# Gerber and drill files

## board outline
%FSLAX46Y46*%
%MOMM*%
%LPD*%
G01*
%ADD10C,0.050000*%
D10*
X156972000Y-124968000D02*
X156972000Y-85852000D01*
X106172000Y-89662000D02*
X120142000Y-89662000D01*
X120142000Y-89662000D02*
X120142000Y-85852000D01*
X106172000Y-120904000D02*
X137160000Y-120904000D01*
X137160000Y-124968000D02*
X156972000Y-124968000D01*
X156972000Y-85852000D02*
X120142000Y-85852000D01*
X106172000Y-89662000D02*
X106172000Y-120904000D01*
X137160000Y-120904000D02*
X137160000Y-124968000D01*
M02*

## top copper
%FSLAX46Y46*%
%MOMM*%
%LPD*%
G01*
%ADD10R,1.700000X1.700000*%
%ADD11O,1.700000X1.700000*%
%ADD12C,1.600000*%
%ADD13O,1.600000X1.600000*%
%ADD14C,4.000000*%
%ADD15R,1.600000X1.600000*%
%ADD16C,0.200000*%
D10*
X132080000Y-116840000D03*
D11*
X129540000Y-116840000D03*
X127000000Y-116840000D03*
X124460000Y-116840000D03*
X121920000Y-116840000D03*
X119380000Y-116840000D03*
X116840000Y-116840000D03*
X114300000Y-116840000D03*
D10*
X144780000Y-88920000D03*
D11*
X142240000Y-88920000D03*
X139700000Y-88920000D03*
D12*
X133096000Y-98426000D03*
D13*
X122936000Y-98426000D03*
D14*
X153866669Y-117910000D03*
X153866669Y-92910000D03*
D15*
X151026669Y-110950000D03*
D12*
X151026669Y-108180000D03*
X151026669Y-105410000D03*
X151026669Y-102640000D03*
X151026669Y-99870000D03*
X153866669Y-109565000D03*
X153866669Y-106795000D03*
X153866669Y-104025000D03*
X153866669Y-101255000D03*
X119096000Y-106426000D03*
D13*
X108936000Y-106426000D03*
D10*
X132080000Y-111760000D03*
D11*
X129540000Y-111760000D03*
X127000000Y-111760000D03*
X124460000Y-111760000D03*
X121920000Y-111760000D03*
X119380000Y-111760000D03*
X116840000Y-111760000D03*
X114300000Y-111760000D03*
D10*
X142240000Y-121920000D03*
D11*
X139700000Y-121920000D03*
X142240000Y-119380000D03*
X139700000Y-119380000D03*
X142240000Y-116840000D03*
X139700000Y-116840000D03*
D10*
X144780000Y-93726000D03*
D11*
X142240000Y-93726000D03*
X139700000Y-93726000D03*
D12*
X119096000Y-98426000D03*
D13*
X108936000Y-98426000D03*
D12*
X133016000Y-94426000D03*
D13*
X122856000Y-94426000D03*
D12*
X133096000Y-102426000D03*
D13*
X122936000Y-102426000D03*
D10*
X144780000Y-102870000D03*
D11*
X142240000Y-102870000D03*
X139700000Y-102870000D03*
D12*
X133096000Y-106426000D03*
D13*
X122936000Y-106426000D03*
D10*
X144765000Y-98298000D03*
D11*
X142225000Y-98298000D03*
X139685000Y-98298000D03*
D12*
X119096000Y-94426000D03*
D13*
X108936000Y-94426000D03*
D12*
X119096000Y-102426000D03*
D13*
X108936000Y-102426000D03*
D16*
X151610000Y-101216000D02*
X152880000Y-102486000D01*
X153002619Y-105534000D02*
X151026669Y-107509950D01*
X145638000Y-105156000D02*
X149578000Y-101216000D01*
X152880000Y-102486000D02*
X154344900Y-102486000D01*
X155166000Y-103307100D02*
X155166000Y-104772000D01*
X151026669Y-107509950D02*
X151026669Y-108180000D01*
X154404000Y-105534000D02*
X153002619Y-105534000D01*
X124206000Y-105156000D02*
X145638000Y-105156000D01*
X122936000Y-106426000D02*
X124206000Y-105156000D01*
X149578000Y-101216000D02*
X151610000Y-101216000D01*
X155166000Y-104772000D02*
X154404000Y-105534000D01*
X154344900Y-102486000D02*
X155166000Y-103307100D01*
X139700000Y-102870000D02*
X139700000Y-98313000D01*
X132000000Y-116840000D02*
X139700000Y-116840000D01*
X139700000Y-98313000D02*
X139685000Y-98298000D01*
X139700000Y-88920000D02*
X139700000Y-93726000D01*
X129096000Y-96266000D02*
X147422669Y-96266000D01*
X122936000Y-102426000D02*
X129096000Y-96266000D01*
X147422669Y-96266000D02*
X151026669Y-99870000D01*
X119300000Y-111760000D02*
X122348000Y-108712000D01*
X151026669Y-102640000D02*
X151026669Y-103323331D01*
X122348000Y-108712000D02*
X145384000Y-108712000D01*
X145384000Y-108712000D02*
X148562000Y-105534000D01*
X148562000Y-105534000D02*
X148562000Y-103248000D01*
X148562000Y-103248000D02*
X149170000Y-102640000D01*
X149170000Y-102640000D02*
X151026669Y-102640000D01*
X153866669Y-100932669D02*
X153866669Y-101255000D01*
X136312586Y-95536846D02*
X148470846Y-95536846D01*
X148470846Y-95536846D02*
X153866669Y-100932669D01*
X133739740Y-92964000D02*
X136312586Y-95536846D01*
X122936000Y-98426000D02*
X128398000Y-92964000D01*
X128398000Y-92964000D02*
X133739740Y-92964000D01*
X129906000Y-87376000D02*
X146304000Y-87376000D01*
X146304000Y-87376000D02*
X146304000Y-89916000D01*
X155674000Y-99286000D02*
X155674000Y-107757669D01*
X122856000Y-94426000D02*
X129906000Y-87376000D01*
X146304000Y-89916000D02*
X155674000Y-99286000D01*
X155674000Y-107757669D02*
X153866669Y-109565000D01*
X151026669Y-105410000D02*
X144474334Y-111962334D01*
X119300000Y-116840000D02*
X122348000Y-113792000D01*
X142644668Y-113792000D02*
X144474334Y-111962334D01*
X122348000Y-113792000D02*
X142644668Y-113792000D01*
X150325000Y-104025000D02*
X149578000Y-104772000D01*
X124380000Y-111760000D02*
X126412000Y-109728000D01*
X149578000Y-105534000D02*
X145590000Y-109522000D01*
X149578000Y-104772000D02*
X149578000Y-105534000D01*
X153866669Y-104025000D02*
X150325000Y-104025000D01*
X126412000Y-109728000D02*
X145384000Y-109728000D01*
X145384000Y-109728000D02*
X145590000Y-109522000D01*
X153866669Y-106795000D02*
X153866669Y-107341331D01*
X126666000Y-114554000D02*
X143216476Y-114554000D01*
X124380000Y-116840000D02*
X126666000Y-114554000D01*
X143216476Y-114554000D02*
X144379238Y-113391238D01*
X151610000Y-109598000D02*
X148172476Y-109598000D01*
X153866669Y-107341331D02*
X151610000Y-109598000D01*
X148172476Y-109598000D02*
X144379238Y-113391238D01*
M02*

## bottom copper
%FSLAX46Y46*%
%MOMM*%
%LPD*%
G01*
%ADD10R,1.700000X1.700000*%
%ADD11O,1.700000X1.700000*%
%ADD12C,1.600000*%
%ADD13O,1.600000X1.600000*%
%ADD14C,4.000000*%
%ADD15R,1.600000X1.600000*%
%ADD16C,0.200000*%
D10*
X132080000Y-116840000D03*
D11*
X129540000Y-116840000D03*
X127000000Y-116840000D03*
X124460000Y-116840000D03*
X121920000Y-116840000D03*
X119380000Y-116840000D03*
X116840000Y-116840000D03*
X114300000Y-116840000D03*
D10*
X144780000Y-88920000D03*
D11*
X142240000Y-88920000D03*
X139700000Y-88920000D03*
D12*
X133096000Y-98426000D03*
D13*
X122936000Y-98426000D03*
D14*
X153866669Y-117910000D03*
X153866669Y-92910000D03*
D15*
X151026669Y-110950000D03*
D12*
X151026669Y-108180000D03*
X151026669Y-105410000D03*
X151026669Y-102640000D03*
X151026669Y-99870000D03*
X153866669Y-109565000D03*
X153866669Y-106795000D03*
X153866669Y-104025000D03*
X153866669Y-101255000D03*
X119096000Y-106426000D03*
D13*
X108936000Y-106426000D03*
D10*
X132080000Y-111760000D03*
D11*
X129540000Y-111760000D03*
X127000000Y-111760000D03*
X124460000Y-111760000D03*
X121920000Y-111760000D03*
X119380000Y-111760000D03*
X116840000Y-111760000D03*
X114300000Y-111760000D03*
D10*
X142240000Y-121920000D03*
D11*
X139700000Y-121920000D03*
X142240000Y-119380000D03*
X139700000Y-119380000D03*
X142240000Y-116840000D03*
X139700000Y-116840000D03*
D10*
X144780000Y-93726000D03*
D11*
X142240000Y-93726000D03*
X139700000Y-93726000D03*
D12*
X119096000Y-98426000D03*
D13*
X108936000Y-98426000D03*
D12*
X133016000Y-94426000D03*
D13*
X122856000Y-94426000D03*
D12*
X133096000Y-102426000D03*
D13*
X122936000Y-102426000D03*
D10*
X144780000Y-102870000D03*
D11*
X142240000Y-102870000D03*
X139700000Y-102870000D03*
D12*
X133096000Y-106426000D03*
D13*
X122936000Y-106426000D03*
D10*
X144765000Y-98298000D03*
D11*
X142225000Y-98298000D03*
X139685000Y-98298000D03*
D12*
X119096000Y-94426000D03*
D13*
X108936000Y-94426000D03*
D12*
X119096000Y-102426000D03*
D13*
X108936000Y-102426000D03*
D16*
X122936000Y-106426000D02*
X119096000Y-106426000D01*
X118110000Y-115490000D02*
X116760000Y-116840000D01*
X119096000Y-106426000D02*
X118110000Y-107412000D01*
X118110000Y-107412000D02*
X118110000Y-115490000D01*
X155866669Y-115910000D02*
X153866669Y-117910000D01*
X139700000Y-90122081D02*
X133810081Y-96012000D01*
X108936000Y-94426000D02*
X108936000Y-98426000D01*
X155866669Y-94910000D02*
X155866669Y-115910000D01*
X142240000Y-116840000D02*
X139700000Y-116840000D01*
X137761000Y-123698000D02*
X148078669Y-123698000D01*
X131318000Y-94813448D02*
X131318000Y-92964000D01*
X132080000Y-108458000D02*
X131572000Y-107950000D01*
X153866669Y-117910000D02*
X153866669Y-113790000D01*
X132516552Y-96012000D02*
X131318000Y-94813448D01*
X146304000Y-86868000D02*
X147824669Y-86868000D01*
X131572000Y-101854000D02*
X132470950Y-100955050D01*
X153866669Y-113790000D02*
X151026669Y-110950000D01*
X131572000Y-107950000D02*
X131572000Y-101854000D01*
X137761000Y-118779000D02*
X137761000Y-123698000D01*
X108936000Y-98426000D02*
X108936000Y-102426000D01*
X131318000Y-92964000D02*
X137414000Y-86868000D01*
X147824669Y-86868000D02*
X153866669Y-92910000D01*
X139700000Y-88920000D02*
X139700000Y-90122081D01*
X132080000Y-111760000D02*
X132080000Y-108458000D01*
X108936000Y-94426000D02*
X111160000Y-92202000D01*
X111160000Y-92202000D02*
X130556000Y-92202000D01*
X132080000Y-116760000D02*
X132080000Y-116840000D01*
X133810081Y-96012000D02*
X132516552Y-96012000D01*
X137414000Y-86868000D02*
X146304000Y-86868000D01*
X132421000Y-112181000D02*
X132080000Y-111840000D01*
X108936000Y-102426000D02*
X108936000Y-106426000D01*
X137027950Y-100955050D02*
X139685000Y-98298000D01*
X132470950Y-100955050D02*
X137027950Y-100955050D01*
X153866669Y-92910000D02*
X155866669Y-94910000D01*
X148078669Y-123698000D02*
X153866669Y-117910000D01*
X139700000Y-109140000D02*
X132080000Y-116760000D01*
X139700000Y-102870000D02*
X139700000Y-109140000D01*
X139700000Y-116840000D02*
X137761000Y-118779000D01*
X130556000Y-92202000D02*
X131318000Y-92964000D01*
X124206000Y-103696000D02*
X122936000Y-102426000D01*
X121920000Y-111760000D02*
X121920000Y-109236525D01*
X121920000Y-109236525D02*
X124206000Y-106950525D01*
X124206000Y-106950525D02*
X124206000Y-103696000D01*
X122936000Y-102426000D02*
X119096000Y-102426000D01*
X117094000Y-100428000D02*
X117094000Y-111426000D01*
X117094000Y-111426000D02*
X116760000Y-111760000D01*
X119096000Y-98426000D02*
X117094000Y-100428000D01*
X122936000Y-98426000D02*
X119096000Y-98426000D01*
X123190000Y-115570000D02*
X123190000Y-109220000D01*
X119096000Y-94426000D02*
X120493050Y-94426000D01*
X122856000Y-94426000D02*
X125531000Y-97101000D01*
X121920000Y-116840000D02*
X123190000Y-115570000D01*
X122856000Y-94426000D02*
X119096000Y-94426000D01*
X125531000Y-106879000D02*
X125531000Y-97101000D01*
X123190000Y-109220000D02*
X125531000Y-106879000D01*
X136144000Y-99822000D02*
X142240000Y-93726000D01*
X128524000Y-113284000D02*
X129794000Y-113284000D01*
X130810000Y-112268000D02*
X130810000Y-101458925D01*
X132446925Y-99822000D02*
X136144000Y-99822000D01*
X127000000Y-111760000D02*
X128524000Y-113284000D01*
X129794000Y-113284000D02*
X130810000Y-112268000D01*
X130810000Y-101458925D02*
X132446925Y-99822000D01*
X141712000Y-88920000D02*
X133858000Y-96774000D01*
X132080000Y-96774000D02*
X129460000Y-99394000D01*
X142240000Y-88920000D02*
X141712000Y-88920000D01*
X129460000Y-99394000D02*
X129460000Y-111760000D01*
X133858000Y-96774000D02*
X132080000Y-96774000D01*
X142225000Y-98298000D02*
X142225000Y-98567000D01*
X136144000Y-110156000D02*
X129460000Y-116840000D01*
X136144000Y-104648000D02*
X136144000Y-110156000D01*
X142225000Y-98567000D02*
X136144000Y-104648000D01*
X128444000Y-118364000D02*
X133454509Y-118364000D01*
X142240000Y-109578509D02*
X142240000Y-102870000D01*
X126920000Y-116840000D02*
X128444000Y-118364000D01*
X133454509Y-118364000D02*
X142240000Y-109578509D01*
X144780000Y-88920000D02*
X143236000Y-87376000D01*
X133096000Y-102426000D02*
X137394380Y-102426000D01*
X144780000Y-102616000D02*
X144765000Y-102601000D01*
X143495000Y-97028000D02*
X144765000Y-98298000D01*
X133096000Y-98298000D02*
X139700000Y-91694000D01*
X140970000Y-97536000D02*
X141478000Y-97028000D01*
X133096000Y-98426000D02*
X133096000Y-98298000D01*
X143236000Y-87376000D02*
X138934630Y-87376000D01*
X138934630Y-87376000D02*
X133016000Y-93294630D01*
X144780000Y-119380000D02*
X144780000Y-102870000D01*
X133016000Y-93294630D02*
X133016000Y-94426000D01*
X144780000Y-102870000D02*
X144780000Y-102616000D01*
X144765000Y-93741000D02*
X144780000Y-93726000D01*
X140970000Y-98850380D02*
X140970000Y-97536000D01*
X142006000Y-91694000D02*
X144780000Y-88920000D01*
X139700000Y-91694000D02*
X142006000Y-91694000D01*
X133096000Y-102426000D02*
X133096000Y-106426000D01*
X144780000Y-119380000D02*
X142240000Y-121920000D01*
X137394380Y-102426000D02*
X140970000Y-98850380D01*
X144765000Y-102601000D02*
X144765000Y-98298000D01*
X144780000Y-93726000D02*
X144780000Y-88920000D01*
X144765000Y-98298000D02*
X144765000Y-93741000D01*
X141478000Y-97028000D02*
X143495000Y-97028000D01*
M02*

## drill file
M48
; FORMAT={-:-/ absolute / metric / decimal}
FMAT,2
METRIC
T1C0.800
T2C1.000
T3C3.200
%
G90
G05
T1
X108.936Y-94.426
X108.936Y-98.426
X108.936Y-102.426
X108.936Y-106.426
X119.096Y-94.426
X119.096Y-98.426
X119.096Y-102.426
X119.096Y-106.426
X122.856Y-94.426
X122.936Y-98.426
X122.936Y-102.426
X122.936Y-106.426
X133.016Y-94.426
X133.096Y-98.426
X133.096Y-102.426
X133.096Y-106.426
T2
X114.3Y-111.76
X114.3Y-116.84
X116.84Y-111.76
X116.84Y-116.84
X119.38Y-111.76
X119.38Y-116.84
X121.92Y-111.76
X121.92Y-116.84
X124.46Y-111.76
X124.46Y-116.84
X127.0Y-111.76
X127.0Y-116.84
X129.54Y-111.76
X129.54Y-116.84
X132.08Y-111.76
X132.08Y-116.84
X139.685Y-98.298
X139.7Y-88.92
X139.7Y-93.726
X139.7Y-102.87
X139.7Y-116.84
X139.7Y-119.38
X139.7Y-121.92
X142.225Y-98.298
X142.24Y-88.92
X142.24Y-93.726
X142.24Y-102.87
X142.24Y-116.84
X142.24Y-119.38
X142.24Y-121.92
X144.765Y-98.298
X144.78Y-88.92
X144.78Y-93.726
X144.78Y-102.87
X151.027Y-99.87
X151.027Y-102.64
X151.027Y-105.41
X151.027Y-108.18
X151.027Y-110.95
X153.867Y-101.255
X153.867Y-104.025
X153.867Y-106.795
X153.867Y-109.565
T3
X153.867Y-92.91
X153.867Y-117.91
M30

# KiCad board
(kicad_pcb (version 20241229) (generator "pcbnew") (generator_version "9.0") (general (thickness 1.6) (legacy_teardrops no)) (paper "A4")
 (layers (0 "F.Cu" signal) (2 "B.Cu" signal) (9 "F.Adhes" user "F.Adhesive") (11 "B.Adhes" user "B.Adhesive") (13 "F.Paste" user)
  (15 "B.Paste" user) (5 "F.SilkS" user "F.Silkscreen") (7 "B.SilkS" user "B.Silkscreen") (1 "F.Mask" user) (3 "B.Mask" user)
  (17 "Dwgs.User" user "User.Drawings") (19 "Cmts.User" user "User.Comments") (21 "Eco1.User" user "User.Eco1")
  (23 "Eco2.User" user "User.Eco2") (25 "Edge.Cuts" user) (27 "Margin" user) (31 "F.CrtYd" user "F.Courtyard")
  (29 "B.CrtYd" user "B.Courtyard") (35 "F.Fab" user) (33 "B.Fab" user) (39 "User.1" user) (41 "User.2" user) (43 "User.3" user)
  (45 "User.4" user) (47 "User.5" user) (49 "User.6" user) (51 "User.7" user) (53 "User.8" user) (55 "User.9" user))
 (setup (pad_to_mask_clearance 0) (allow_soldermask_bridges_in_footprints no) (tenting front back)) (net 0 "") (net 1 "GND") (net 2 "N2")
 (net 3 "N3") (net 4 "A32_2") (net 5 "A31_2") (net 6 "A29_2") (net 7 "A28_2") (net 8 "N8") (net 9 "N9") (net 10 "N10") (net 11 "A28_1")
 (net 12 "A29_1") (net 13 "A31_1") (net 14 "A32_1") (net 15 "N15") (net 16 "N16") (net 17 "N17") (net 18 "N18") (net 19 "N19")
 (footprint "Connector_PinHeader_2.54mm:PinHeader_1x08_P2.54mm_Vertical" (layer "F.Cu") (at 132.08 116.84 -90)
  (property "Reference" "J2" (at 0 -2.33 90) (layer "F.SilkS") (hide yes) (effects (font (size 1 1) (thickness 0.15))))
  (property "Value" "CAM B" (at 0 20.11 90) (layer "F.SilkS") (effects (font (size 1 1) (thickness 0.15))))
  (pad "1" thru_hole rect (at 0 0 270) (size 1.7 1.7) (drill 1) (layers "*.Cu" "*.Mask") (remove_unused_layers no) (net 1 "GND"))
  (pad "2" thru_hole oval (at 0 2.54 270) (size 1.7 1.7) (drill 1) (layers "*.Cu" "*.Mask") (remove_unused_layers no) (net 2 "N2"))
  (pad "3" thru_hole oval (at 0 5.08 270) (size 1.7 1.7) (drill 1) (layers "*.Cu" "*.Mask") (remove_unused_layers no) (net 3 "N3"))
  (pad "4" thru_hole oval (at 0 7.62 270) (size 1.7 1.7) (drill 1) (layers "*.Cu" "*.Mask") (remove_unused_layers no) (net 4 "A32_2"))
  (pad "5" thru_hole oval (at 0 10.16 270) (size 1.7 1.7) (drill 1) (layers "*.Cu" "*.Mask") (remove_unused_layers no) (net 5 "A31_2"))
  (pad "6" thru_hole oval (at 0 12.7 270) (size 1.7 1.7) (drill 1) (layers "*.Cu" "*.Mask") (remove_unused_layers no) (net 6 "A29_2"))
  (pad "7" thru_hole oval (at 0 15.24 270) (size 1.7 1.7) (drill 1) (layers "*.Cu" "*.Mask") (remove_unused_layers no) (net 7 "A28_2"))
  (pad "8" thru_hole oval (at 0 17.78 270) (size 1.7 1.7) (drill 1) (layers "*.Cu" "*.Mask") (remove_unused_layers no) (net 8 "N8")))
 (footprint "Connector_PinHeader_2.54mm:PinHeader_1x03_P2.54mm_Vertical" (layer "F.Cu") (at 144.78 88.92 -90)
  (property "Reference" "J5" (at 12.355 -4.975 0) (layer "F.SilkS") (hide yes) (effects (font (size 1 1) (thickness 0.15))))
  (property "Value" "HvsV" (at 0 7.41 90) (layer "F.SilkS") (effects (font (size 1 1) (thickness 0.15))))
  (pad "1" thru_hole rect (at 0 0 270) (size 1.7 1.7) (drill 1) (layers "*.Cu" "*.Mask") (remove_unused_layers no) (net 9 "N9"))
  (pad "2" thru_hole oval (at 0 2.54 270) (size 1.7 1.7) (drill 1) (layers "*.Cu" "*.Mask") (remove_unused_layers no) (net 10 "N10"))
  (pad "3" thru_hole oval (at 0 5.08 270) (size 1.7 1.7) (drill 1) (layers "*.Cu" "*.Mask") (remove_unused_layers no) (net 1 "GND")))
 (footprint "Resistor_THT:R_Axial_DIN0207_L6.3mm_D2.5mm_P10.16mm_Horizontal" (layer "F.Cu") (at 133.096 98.426 180)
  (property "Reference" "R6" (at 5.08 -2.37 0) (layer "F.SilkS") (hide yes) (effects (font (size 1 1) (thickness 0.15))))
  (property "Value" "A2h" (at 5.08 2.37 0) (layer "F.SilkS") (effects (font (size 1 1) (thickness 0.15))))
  (pad "1" thru_hole circle (at 0 0 180) (size 1.6 1.6) (drill 0.8) (layers "*.Cu" "*.Mask") (remove_unused_layers no) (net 9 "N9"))
  (pad "2" thru_hole oval (at 10.16 0 180) (size 1.6 1.6) (drill 0.8) (layers "*.Cu" "*.Mask") (remove_unused_layers no) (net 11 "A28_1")))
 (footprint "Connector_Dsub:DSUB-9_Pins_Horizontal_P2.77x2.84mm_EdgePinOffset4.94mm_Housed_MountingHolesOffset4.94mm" (layer "F.Cu")
  (at 151.026669 110.95 90)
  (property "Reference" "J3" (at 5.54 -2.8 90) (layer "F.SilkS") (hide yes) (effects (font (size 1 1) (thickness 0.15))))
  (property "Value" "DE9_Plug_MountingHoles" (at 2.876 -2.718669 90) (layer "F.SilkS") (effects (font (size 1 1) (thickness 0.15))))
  (pad "0" thru_hole circle (at -6.96 2.84 90) (size 4 4) (drill 3.2) (layers "*.Cu" "*.Mask") (remove_unused_layers no) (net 1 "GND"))
  (pad "0" thru_hole circle (at 18.04 2.84 90) (size 4 4) (drill 3.2) (layers "*.Cu" "*.Mask") (remove_unused_layers no) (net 1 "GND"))
  (pad "1" thru_hole rect (at 0 0 90) (size 1.6 1.6) (drill 1) (layers "*.Cu" "*.Mask") (remove_unused_layers no) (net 1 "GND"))
  (pad "2" thru_hole circle (at 2.77 0 90) (size 1.6 1.6) (drill 1) (layers "*.Cu" "*.Mask") (remove_unused_layers no) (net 7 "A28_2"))
  (pad "3" thru_hole circle (at 5.54 0 90) (size 1.6 1.6) (drill 1) (layers "*.Cu" "*.Mask") (remove_unused_layers no) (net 6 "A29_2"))
  (pad "4" thru_hole circle (at 8.31 0 90) (size 1.6 1.6) (drill 1) (layers "*.Cu" "*.Mask") (remove_unused_layers no) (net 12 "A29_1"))
  (pad "5" thru_hole circle (at 11.08 0 90) (size 1.6 1.6) (drill 1) (layers "*.Cu" "*.Mask") (remove_unused_layers no) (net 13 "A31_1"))
  (pad "6" thru_hole circle (at 1.385 2.84 90) (size 1.6 1.6) (drill 1) (layers "*.Cu" "*.Mask") (remove_unused_layers no) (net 5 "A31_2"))
  (pad "7" thru_hole circle (at 4.155 2.84 90) (size 1.6 1.6) (drill 1) (layers "*.Cu" "*.Mask") (remove_unused_layers no) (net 4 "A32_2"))
  (pad "8" thru_hole circle (at 6.925 2.84 90) (size 1.6 1.6) (drill 1) (layers "*.Cu" "*.Mask") (remove_unused_layers no) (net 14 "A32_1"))
  (pad "9" thru_hole circle (at 9.695 2.84 90) (size 1.6 1.6) (drill 1) (layers "*.Cu" "*.Mask") (remove_unused_layers no) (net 11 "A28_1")))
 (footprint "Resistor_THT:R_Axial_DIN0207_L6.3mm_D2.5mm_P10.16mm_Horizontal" (layer "F.Cu") (at 119.096 106.426 180)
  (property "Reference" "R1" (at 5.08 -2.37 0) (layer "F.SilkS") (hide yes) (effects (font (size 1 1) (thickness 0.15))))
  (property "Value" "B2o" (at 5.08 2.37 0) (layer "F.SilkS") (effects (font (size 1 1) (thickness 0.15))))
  (pad "1" thru_hole circle (at 0 0 180) (size 1.6 1.6) (drill 0.8) (layers "*.Cu" "*.Mask") (remove_unused_layers no) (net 7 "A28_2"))
  (pad "2" thru_hole oval (at 10.16 0 180) (size 1.6 1.6) (drill 0.8) (layers "*.Cu" "*.Mask") (remove_unused_layers no) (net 1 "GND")))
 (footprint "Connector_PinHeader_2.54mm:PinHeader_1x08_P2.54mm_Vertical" (layer "F.Cu") (at 132.08 111.76 -90)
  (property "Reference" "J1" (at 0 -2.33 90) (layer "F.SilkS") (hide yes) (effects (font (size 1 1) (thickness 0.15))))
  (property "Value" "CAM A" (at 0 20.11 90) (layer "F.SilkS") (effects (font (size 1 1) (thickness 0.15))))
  (pad "1" thru_hole rect (at 0 0 270) (size 1.7 1.7) (drill 1) (layers "*.Cu" "*.Mask") (remove_unused_layers no) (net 1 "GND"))
  (pad "2" thru_hole oval (at 0 2.54 270) (size 1.7 1.7) (drill 1) (layers "*.Cu" "*.Mask") (remove_unused_layers no) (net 10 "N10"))
  (pad "3" thru_hole oval (at 0 5.08 270) (size 1.7 1.7) (drill 1) (layers "*.Cu" "*.Mask") (remove_unused_layers no) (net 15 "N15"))
  (pad "4" thru_hole oval (at 0 7.62 270) (size 1.7 1.7) (drill 1) (layers "*.Cu" "*.Mask") (remove_unused_layers no) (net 14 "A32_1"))
  (pad "5" thru_hole oval (at 0 10.16 270) (size 1.7 1.7) (drill 1) (layers "*.Cu" "*.Mask") (remove_unused_layers no) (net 13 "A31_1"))
  (pad "6" thru_hole oval (at 0 12.7 270) (size 1.7 1.7) (drill 1) (layers "*.Cu" "*.Mask") (remove_unused_layers no) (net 12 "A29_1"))
  (pad "7" thru_hole oval (at 0 15.24 270) (size 1.7 1.7) (drill 1) (layers "*.Cu" "*.Mask") (remove_unused_layers no) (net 11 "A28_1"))
  (pad "8" thru_hole oval (at 0 17.78 270) (size 1.7 1.7) (drill 1) (layers "*.Cu" "*.Mask") (remove_unused_layers no) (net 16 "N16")))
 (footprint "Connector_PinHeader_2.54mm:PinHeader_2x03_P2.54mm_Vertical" (layer "F.Cu") (at 142.24 121.92 180)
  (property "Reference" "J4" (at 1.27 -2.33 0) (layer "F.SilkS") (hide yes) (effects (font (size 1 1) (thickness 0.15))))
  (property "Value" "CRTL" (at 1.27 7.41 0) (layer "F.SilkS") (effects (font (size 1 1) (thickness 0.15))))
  (pad "1" thru_hole rect (at 0 0 180) (size 1.7 1.7) (drill 1) (layers "*.Cu" "*.Mask") (remove_unused_layers no) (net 9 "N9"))
  (pad "2" thru_hole oval (at 2.54 0 180) (size 1.7 1.7) (drill 1) (layers "*.Cu" "*.Mask") (remove_unused_layers no) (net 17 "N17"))
  (pad "3" thru_hole oval (at 0 2.54 180) (size 1.7 1.7) (drill 1) (layers "*.Cu" "*.Mask") (remove_unused_layers no) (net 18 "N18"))
  (pad "4" thru_hole oval (at 2.54 2.54 180) (size 1.7 1.7) (drill 1) (layers "*.Cu" "*.Mask") (remove_unused_layers no) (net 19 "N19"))
  (pad "5" thru_hole oval (at 0 5.08 180) (size 1.7 1.7) (drill 1) (layers "*.Cu" "*.Mask") (remove_unused_layers no) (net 1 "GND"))
  (pad "6" thru_hole oval (at 2.54 5.08 180) (size 1.7 1.7) (drill 1) (layers "*.Cu" "*.Mask") (remove_unused_layers no) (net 1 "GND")))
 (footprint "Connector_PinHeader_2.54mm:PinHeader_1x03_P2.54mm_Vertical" (layer "F.Cu") (at 144.78 93.726 -90)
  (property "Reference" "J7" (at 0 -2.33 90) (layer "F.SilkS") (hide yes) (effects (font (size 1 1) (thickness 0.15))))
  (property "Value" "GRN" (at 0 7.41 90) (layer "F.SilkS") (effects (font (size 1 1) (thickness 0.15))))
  (pad "1" thru_hole rect (at 0 0 270) (size 1.7 1.7) (drill 1) (layers "*.Cu" "*.Mask") (remove_unused_layers no) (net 9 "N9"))
  (pad "2" thru_hole oval (at 0 2.54 270) (size 1.7 1.7) (drill 1) (layers "*.Cu" "*.Mask") (remove_unused_layers no) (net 15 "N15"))
  (pad "3" thru_hole oval (at 0 5.08 270) (size 1.7 1.7) (drill 1) (layers "*.Cu" "*.Mask") (remove_unused_layers no) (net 1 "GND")))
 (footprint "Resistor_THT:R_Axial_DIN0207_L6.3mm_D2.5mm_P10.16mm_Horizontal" (layer "F.Cu") (at 119.096 98.426 180)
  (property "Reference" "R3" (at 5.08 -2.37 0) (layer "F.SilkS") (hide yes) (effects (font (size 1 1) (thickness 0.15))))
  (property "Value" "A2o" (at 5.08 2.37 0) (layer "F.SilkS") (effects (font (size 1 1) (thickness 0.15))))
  (pad "1" thru_hole circle (at 0 0 180) (size 1.6 1.6) (drill 0.8) (layers "*.Cu" "*.Mask") (remove_unused_layers no) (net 11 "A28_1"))
  (pad "2" thru_hole oval (at 10.16 0 180) (size 1.6 1.6) (drill 0.8) (layers "*.Cu" "*.Mask") (remove_unused_layers no) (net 1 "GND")))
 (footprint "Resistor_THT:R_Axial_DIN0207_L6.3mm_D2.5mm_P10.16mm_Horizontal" (layer "F.Cu") (at 133.016 94.426 180)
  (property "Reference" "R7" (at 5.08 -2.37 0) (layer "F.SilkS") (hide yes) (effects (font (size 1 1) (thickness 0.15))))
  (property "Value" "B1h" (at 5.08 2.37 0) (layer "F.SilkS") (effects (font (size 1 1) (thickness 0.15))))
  (pad "1" thru_hole circle (at 0 0 180) (size 1.6 1.6) (drill 0.8) (layers "*.Cu" "*.Mask") (remove_unused_layers no) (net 9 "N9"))
  (pad "2" thru_hole oval (at 10.16 0 180) (size 1.6 1.6) (drill 0.8) (layers "*.Cu" "*.Mask") (remove_unused_layers no) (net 5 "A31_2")))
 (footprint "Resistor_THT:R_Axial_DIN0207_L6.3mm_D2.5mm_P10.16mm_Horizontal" (layer "F.Cu") (at 133.096 102.426 180)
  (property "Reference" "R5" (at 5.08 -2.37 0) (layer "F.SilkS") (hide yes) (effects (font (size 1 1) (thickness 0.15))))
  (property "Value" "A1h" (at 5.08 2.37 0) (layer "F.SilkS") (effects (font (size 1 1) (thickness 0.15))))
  (pad "1" thru_hole circle (at 0 0 180) (size 1.6 1.6) (drill 0.8) (layers "*.Cu" "*.Mask") (remove_unused_layers no) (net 9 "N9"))
  (pad "2" thru_hole oval (at 10.16 0 180) (size 1.6 1.6) (drill 0.8) (layers "*.Cu" "*.Mask") (remove_unused_layers no) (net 13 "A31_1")))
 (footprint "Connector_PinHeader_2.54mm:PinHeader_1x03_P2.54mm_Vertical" (layer "F.Cu") (at 144.78 102.87 -90)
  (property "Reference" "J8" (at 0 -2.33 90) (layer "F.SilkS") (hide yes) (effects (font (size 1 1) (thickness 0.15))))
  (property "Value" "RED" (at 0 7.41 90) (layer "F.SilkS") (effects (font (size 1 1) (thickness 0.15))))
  (pad "1" thru_hole rect (at 0 0 270) (size 1.7 1.7) (drill 1) (layers "*.Cu" "*.Mask") (remove_unused_layers no) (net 9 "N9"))
  (pad "2" thru_hole oval (at 0 2.54 270) (size 1.7 1.7) (drill 1) (layers "*.Cu" "*.Mask") (remove_unused_layers no) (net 3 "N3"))
  (pad "3" thru_hole oval (at 0 5.08 270) (size 1.7 1.7) (drill 1) (layers "*.Cu" "*.Mask") (remove_unused_layers no) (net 1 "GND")))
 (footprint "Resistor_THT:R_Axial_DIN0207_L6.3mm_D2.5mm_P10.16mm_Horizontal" (layer "F.Cu") (at 133.096 106.426 180)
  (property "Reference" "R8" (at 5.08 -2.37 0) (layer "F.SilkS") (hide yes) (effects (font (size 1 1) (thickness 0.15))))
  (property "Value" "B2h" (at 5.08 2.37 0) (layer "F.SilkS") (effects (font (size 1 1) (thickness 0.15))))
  (pad "1" thru_hole circle (at 0 0 180) (size 1.6 1.6) (drill 0.8) (layers "*.Cu" "*.Mask") (remove_unused_layers no) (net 9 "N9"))
  (pad "2" thru_hole oval (at 10.16 0 180) (size 1.6 1.6) (drill 0.8) (layers "*.Cu" "*.Mask") (remove_unused_layers no) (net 7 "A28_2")))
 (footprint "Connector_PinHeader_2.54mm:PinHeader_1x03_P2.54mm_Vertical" (layer "F.Cu") (at 144.765 98.298 -90)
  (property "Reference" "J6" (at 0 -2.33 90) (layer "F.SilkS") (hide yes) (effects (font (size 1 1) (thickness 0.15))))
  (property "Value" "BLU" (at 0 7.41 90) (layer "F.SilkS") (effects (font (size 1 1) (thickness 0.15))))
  (pad "1" thru_hole rect (at 0 0 270) (size 1.7 1.7) (drill 1) (layers "*.Cu" "*.Mask") (remove_unused_layers no) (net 9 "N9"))
  (pad "2" thru_hole oval (at 0 2.54 270) (size 1.7 1.7) (drill 1) (layers "*.Cu" "*.Mask") (remove_unused_layers no) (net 2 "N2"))
  (pad "3" thru_hole oval (at 0 5.08 270) (size 1.7 1.7) (drill 1) (layers "*.Cu" "*.Mask") (remove_unused_layers no) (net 1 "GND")))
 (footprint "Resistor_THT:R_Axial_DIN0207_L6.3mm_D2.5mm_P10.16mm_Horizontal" (layer "F.Cu") (at 119.096 94.426 180)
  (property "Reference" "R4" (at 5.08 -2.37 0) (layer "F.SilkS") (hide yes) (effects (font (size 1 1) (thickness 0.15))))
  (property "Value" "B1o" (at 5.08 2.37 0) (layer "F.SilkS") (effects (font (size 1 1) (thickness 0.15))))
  (pad "1" thru_hole circle (at 0 0 180) (size 1.6 1.6) (drill 0.8) (layers "*.Cu" "*.Mask") (remove_unused_layers no) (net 5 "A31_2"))
  (pad "2" thru_hole oval (at 10.16 0 180) (size 1.6 1.6) (drill 0.8) (layers "*.Cu" "*.Mask") (remove_unused_layers no) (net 1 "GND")))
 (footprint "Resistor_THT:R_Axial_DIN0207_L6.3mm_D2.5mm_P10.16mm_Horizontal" (layer "F.Cu") (at 119.096 102.426 180)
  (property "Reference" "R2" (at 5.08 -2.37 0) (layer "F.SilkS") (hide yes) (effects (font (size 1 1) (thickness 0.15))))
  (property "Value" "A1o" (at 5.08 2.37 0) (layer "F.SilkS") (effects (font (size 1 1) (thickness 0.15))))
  (pad "1" thru_hole circle (at 0 0 180) (size 1.6 1.6) (drill 0.8) (layers "*.Cu" "*.Mask") (remove_unused_layers no) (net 13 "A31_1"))
  (pad "2" thru_hole oval (at 10.16 0 180) (size 1.6 1.6) (drill 0.8) (layers "*.Cu" "*.Mask") (remove_unused_layers no) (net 1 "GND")))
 (gr_line (start 156.972 124.968) (end 156.972 85.852) (stroke (width 0.05) (type default)) (layer "Edge.Cuts"))
 (gr_line (start 106.172 89.662) (end 120.142 89.662) (stroke (width 0.05) (type default)) (layer "Edge.Cuts"))
 (gr_line (start 120.142 89.662) (end 120.142 85.852) (stroke (width 0.05) (type default)) (layer "Edge.Cuts"))
 (gr_line (start 106.172 120.904) (end 137.16 120.904) (stroke (width 0.05) (type default)) (layer "Edge.Cuts"))
 (gr_line (start 137.16 124.968) (end 156.972 124.968) (stroke (width 0.05) (type default)) (layer "Edge.Cuts"))
 (gr_line (start 156.972 85.852) (end 120.142 85.852) (stroke (width 0.05) (type default)) (layer "Edge.Cuts"))
 (gr_line (start 106.172 89.662) (end 106.172 120.904) (stroke (width 0.05) (type default)) (layer "Edge.Cuts"))
 (gr_line (start 137.16 120.904) (end 137.16 124.968) (stroke (width 0.05) (type default)) (layer "Edge.Cuts"))
 (segment (start 151.61 101.216) (end 152.88 102.486) (width 0.2) (layer "F.Cu") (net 7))
 (segment (start 153.002619 105.534) (end 151.026669 107.50995) (width 0.2) (layer "F.Cu") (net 7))
 (segment (start 145.638 105.156) (end 149.578 101.216) (width 0.2) (layer "F.Cu") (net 7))
 (segment (start 152.88 102.486) (end 154.3449 102.486) (width 0.2) (layer "F.Cu") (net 7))
 (segment (start 155.166 103.3071) (end 155.166 104.772) (width 0.2) (layer "F.Cu") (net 7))
 (segment (start 151.026669 107.50995) (end 151.026669 108.18) (width 0.2) (layer "F.Cu") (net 7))
 (segment (start 154.404 105.534) (end 153.002619 105.534) (width 0.2) (layer "F.Cu") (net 7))
 (segment (start 124.206 105.156) (end 145.638 105.156) (width 0.2) (layer "F.Cu") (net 7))
 (segment (start 122.936 106.426) (end 124.206 105.156) (width 0.2) (layer "F.Cu") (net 7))
 (segment (start 149.578 101.216) (end 151.61 101.216) (width 0.2) (layer "F.Cu") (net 7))
 (segment (start 155.166 104.772) (end 154.404 105.534) (width 0.2) (layer "F.Cu") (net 7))
 (segment (start 154.3449 102.486) (end 155.166 103.3071) (width 0.2) (layer "F.Cu") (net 7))
 (segment (start 122.936 106.426) (end 119.096 106.426) (width 0.2) (layer "B.Cu") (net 7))
 (segment (start 118.11 115.49) (end 116.76 116.84) (width 0.2) (layer "B.Cu") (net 7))
 (segment (start 119.096 106.426) (end 118.11 107.412) (width 0.2) (layer "B.Cu") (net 7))
 (segment (start 118.11 107.412) (end 118.11 115.49) (width 0.2) (layer "B.Cu") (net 7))
 (segment (start 139.7 102.87) (end 139.7 98.313) (width 0.2) (layer "F.Cu") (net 1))
 (segment (start 132 116.84) (end 139.7 116.84) (width 0.2) (layer "F.Cu") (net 1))
 (segment (start 139.7 98.313) (end 139.685 98.298) (width 0.2) (layer "F.Cu") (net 1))
 (segment (start 139.7 88.92) (end 139.7 93.726) (width 0.2) (layer "F.Cu") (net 1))
 (segment (start 155.866669 115.91) (end 153.866669 117.91) (width 0.2) (layer "B.Cu") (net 1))
 (segment (start 139.7 90.122081) (end 133.810081 96.012) (width 0.2) (layer "B.Cu") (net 1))
 (segment (start 108.936 94.426) (end 108.936 98.426) (width 0.2) (layer "B.Cu") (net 1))
 (segment (start 155.866669 94.91) (end 155.866669 115.91) (width 0.2) (layer "B.Cu") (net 1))
 (segment (start 142.24 116.84) (end 139.7 116.84) (width 0.2) (layer "B.Cu") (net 1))
 (segment (start 137.761 123.698) (end 148.078669 123.698) (width 0.2) (layer "B.Cu") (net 1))
 (segment (start 131.318 94.813448) (end 131.318 92.964) (width 0.2) (layer "B.Cu") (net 1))
 (segment (start 132.08 108.458) (end 131.572 107.95) (width 0.2) (layer "B.Cu") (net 1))
 (segment (start 153.866669 117.91) (end 153.866669 113.79) (width 0.2) (layer "B.Cu") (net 1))
 (segment (start 132.516552 96.012) (end 131.318 94.813448) (width 0.2) (layer "B.Cu") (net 1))
 (segment (start 146.304 86.868) (end 147.824669 86.868) (width 0.2) (layer "B.Cu") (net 1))
 (segment (start 131.572 101.854) (end 132.47095 100.95505) (width 0.2) (layer "B.Cu") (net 1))
 (segment (start 153.866669 113.79) (end 151.026669 110.95) (width 0.2) (layer "B.Cu") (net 1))
 (segment (start 131.572 107.95) (end 131.572 101.854) (width 0.2) (layer "B.Cu") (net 1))
 (segment (start 137.761 118.779) (end 137.761 123.698) (width 0.2) (layer "B.Cu") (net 1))
 (segment (start 108.936 98.426) (end 108.936 102.426) (width 0.2) (layer "B.Cu") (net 1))
 (segment (start 131.318 92.964) (end 137.414 86.868) (width 0.2) (layer "B.Cu") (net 1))
 (segment (start 147.824669 86.868) (end 153.866669 92.91) (width 0.2) (layer "B.Cu") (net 1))
 (segment (start 139.7 88.92) (end 139.7 90.122081) (width 0.2) (layer "B.Cu") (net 1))
 (segment (start 132.08 111.76) (end 132.08 108.458) (width 0.2) (layer "B.Cu") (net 1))
 (segment (start 108.936 94.426) (end 111.16 92.202) (width 0.2) (layer "B.Cu") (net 1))
 (segment (start 111.16 92.202) (end 130.556 92.202) (width 0.2) (layer "B.Cu") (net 1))
 (segment (start 132.08 116.76) (end 132.08 116.84) (width 0.2) (layer "B.Cu") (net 1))
 (segment (start 133.810081 96.012) (end 132.516552 96.012) (width 0.2) (layer "B.Cu") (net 1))
 (segment (start 137.414 86.868) (end 146.304 86.868) (width 0.2) (layer "B.Cu") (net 1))
 (segment (start 132.421 112.181) (end 132.08 111.84) (width 0.2) (layer "B.Cu") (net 1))
 (segment (start 108.936 102.426) (end 108.936 106.426) (width 0.2) (layer "B.Cu") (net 1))
 (segment (start 137.02795 100.95505) (end 139.685 98.298) (width 0.2) (layer "B.Cu") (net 1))
 (segment (start 132.47095 100.95505) (end 137.02795 100.95505) (width 0.2) (layer "B.Cu") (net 1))
 (segment (start 153.866669 92.91) (end 155.866669 94.91) (width 0.2) (layer "B.Cu") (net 1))
 (segment (start 148.078669 123.698) (end 153.866669 117.91) (width 0.2) (layer "B.Cu") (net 1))
 (segment (start 139.7 109.14) (end 132.08 116.76) (width 0.2) (layer "B.Cu") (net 1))
 (segment (start 139.7 102.87) (end 139.7 109.14) (width 0.2) (layer "B.Cu") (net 1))
 (segment (start 139.7 116.84) (end 137.761 118.779) (width 0.2) (layer "B.Cu") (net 1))
 (segment (start 130.556 92.202) (end 131.318 92.964) (width 0.2) (layer "B.Cu") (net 1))
 (segment (start 129.096 96.266) (end 147.422669 96.266) (width 0.2) (layer "F.Cu") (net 13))
 (segment (start 122.936 102.426) (end 129.096 96.266) (width 0.2) (layer "F.Cu") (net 13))
 (segment (start 147.422669 96.266) (end 151.026669 99.87) (width 0.2) (layer "F.Cu") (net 13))
 (segment (start 124.206 103.696) (end 122.936 102.426) (width 0.2) (layer "B.Cu") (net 13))
 (segment (start 121.92 111.76) (end 121.92 109.236525) (width 0.2) (layer "B.Cu") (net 13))
 (segment (start 121.92 109.236525) (end 124.206 106.950525) (width 0.2) (layer "B.Cu") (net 13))
 (segment (start 124.206 106.950525) (end 124.206 103.696) (width 0.2) (layer "B.Cu") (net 13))
 (segment (start 122.936 102.426) (end 119.096 102.426) (width 0.2) (layer "B.Cu") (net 13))
 (segment (start 119.3 111.76) (end 122.348 108.712) (width 0.2) (layer "F.Cu") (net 12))
 (segment (start 151.026669 102.64) (end 151.026669 103.323331) (width 0.2) (layer "F.Cu") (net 12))
 (segment (start 122.348 108.712) (end 145.384 108.712) (width 0.2) (layer "F.Cu") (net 12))
 (segment (start 145.384 108.712) (end 148.562 105.534) (width 0.2) (layer "F.Cu") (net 12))
 (segment (start 148.562 105.534) (end 148.562 103.248) (width 0.2) (layer "F.Cu") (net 12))
 (segment (start 148.562 103.248) (end 149.17 102.64) (width 0.2) (layer "F.Cu") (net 12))
 (segment (start 149.17 102.64) (end 151.026669 102.64) (width 0.2) (layer "F.Cu") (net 12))
 (segment (start 153.866669 100.932669) (end 153.866669 101.255) (width 0.2) (layer "F.Cu") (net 11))
 (segment (start 136.312586 95.536846) (end 148.470846 95.536846) (width 0.2) (layer "F.Cu") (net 11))
 (segment (start 148.470846 95.536846) (end 153.866669 100.932669) (width 0.2) (layer "F.Cu") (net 11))
 (segment (start 133.73974 92.964) (end 136.312586 95.536846) (width 0.2) (layer "F.Cu") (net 11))
 (segment (start 122.936 98.426) (end 128.398 92.964) (width 0.2) (layer "F.Cu") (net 11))
 (segment (start 128.398 92.964) (end 133.73974 92.964) (width 0.2) (layer "F.Cu") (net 11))
 (segment (start 117.094 100.428) (end 117.094 111.426) (width 0.2) (layer "B.Cu") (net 11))
 (segment (start 117.094 111.426) (end 116.76 111.76) (width 0.2) (layer "B.Cu") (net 11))
 (segment (start 119.096 98.426) (end 117.094 100.428) (width 0.2) (layer "B.Cu") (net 11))
 (segment (start 122.936 98.426) (end 119.096 98.426) (width 0.2) (layer "B.Cu") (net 11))
 (segment (start 129.906 87.376) (end 146.304 87.376) (width 0.2) (layer "F.Cu") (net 5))
 (segment (start 146.304 87.376) (end 146.304 89.916) (width 0.2) (layer "F.Cu") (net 5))
 (segment (start 155.674 99.286) (end 155.674 107.757669) (width 0.2) (layer "F.Cu") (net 5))
 (segment (start 122.856 94.426) (end 129.906 87.376) (width 0.2) (layer "F.Cu") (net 5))
 (segment (start 146.304 89.916) (end 155.674 99.286) (width 0.2) (layer "F.Cu") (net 5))
 (segment (start 155.674 107.757669) (end 153.866669 109.565) (width 0.2) (layer "F.Cu") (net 5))
 (segment (start 123.19 115.57) (end 123.19 109.22) (width 0.2) (layer "B.Cu") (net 5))
 (segment (start 119.096 94.426) (end 120.49305 94.426) (width 0.2) (layer "B.Cu") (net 5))
 (segment (start 122.856 94.426) (end 125.531 97.101) (width 0.2) (layer "B.Cu") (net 5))
 (segment (start 121.92 116.84) (end 123.19 115.57) (width 0.2) (layer "B.Cu") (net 5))
 (segment (start 122.856 94.426) (end 119.096 94.426) (width 0.2) (layer "B.Cu") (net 5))
 (segment (start 125.531 106.879) (end 125.531 97.101) (width 0.2) (layer "B.Cu") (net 5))
 (segment (start 123.19 109.22) (end 125.531 106.879) (width 0.2) (layer "B.Cu") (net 5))
 (segment (start 151.026669 105.41) (end 144.474334 111.962334) (width 0.2) (layer "F.Cu") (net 6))
 (segment (start 119.3 116.84) (end 122.348 113.792) (width 0.2) (layer "F.Cu") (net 6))
 (segment (start 142.644668 113.792) (end 144.474334 111.962334) (width 0.2) (layer "F.Cu") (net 6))
 (segment (start 122.348 113.792) (end 142.644668 113.792) (width 0.2) (layer "F.Cu") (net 6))
 (segment (start 150.325 104.025) (end 149.578 104.772) (width 0.2) (layer "F.Cu") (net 14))
 (segment (start 124.38 111.76) (end 126.412 109.728) (width 0.2) (layer "F.Cu") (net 14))
 (segment (start 149.578 105.534) (end 145.59 109.522) (width 0.2) (layer "F.Cu") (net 14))
 (segment (start 149.578 104.772) (end 149.578 105.534) (width 0.2) (layer "F.Cu") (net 14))
 (segment (start 153.866669 104.025) (end 150.325 104.025) (width 0.2) (layer "F.Cu") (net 14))
 (segment (start 126.412 109.728) (end 145.384 109.728) (width 0.2) (layer "F.Cu") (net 14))
 (segment (start 145.384 109.728) (end 145.59 109.522) (width 0.2) (layer "F.Cu") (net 14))
 (segment (start 136.144 99.822) (end 142.24 93.726) (width 0.2) (layer "B.Cu") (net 15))
 (segment (start 128.524 113.284) (end 129.794 113.284) (width 0.2) (layer "B.Cu") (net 15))
 (segment (start 130.81 112.268) (end 130.81 101.458925) (width 0.2) (layer "B.Cu") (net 15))
 (segment (start 132.446925 99.822) (end 136.144 99.822) (width 0.2) (layer "B.Cu") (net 15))
 (segment (start 127 111.76) (end 128.524 113.284) (width 0.2) (layer "B.Cu") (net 15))
 (segment (start 129.794 113.284) (end 130.81 112.268) (width 0.2) (layer "B.Cu") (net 15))
 (segment (start 130.81 101.458925) (end 132.446925 99.822) (width 0.2) (layer "B.Cu") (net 15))
 (segment (start 141.712 88.92) (end 133.858 96.774) (width 0.2) (layer "B.Cu") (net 10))
 (segment (start 132.08 96.774) (end 129.46 99.394) (width 0.2) (layer "B.Cu") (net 10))
 (segment (start 142.24 88.92) (end 141.712 88.92) (width 0.2) (layer "B.Cu") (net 10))
 (segment (start 129.46 99.394) (end 129.46 111.76) (width 0.2) (layer "B.Cu") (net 10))
 (segment (start 133.858 96.774) (end 132.08 96.774) (width 0.2) (layer "B.Cu") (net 10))
 (segment (start 142.225 98.298) (end 142.225 98.567) (width 0.2) (layer "B.Cu") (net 2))
 (segment (start 136.144 110.156) (end 129.46 116.84) (width 0.2) (layer "B.Cu") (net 2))
 (segment (start 136.144 104.648) (end 136.144 110.156) (width 0.2) (layer "B.Cu") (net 2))
 (segment (start 142.225 98.567) (end 136.144 104.648) (width 0.2) (layer "B.Cu") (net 2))
 (segment (start 128.444 118.364) (end 133.454509 118.364) (width 0.2) (layer "B.Cu") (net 3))
 (segment (start 142.24 109.578509) (end 142.24 102.87) (width 0.2) (layer "B.Cu") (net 3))
 (segment (start 126.92 116.84) (end 128.444 118.364) (width 0.2) (layer "B.Cu") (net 3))
 (segment (start 133.454509 118.364) (end 142.24 109.578509) (width 0.2) (layer "B.Cu") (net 3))
 (segment (start 153.866669 106.795) (end 153.866669 107.341331) (width 0.2) (layer "F.Cu") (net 4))
 (segment (start 126.666 114.554) (end 143.216476 114.554) (width 0.2) (layer "F.Cu") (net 4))
 (segment (start 124.38 116.84) (end 126.666 114.554) (width 0.2) (layer "F.Cu") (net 4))
 (segment (start 143.216476 114.554) (end 144.379238 113.391238) (width 0.2) (layer "F.Cu") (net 4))
 (segment (start 151.61 109.598) (end 148.172476 109.598) (width 0.2) (layer "F.Cu") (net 4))
 (segment (start 153.866669 107.341331) (end 151.61 109.598) (width 0.2) (layer "F.Cu") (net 4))
 (segment (start 148.172476 109.598) (end 144.379238 113.391238) (width 0.2) (layer "F.Cu") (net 4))
 (segment (start 144.78 88.92) (end 143.236 87.376) (width 0.2) (layer "B.Cu") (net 9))
 (segment (start 133.096 102.426) (end 137.39438 102.426) (width 0.2) (layer "B.Cu") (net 9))
 (segment (start 144.78 102.616) (end 144.765 102.601) (width 0.2) (layer "B.Cu") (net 9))
 (segment (start 143.495 97.028) (end 144.765 98.298) (width 0.2) (layer "B.Cu") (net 9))
 (segment (start 133.096 98.298) (end 139.7 91.694) (width 0.2) (layer "B.Cu") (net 9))
 (segment (start 140.97 97.536) (end 141.478 97.028) (width 0.2) (layer "B.Cu") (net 9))
 (segment (start 133.096 98.426) (end 133.096 98.298) (width 0.2) (layer "B.Cu") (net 9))
 (segment (start 143.236 87.376) (end 138.93463 87.376) (width 0.2) (layer "B.Cu") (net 9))
 (segment (start 138.93463 87.376) (end 133.016 93.29463) (width 0.2) (layer "B.Cu") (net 9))
 (segment (start 144.78 119.38) (end 144.78 102.87) (width 0.2) (layer "B.Cu") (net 9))
 (segment (start 133.016 93.29463) (end 133.016 94.426) (width 0.2) (layer "B.Cu") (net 9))
 (segment (start 144.78 102.87) (end 144.78 102.616) (width 0.2) (layer "B.Cu") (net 9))
 (segment (start 144.765 93.741) (end 144.78 93.726) (width 0.2) (layer "B.Cu") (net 9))
 (segment (start 140.97 98.85038) (end 140.97 97.536) (width 0.2) (layer "B.Cu") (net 9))
 (segment (start 142.006 91.694) (end 144.78 88.92) (width 0.2) (layer "B.Cu") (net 9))
 (segment (start 139.7 91.694) (end 142.006 91.694) (width 0.2) (layer "B.Cu") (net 9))
 (segment (start 133.096 102.426) (end 133.096 106.426) (width 0.2) (layer "B.Cu") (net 9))
 (segment (start 144.78 119.38) (end 142.24 121.92) (width 0.2) (layer "B.Cu") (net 9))
 (segment (start 137.39438 102.426) (end 140.97 98.85038) (width 0.2) (layer "B.Cu") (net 9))
 (segment (start 144.765 102.601) (end 144.765 98.298) (width 0.2) (layer "B.Cu") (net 9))
 (segment (start 144.78 93.726) (end 144.78 88.92) (width 0.2) (layer "B.Cu") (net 9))
 (segment (start 144.765 98.298) (end 144.765 93.741) (width 0.2) (layer "B.Cu") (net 9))
 (segment (start 141.478 97.028) (end 143.495 97.028) (width 0.2) (layer "B.Cu") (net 9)))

